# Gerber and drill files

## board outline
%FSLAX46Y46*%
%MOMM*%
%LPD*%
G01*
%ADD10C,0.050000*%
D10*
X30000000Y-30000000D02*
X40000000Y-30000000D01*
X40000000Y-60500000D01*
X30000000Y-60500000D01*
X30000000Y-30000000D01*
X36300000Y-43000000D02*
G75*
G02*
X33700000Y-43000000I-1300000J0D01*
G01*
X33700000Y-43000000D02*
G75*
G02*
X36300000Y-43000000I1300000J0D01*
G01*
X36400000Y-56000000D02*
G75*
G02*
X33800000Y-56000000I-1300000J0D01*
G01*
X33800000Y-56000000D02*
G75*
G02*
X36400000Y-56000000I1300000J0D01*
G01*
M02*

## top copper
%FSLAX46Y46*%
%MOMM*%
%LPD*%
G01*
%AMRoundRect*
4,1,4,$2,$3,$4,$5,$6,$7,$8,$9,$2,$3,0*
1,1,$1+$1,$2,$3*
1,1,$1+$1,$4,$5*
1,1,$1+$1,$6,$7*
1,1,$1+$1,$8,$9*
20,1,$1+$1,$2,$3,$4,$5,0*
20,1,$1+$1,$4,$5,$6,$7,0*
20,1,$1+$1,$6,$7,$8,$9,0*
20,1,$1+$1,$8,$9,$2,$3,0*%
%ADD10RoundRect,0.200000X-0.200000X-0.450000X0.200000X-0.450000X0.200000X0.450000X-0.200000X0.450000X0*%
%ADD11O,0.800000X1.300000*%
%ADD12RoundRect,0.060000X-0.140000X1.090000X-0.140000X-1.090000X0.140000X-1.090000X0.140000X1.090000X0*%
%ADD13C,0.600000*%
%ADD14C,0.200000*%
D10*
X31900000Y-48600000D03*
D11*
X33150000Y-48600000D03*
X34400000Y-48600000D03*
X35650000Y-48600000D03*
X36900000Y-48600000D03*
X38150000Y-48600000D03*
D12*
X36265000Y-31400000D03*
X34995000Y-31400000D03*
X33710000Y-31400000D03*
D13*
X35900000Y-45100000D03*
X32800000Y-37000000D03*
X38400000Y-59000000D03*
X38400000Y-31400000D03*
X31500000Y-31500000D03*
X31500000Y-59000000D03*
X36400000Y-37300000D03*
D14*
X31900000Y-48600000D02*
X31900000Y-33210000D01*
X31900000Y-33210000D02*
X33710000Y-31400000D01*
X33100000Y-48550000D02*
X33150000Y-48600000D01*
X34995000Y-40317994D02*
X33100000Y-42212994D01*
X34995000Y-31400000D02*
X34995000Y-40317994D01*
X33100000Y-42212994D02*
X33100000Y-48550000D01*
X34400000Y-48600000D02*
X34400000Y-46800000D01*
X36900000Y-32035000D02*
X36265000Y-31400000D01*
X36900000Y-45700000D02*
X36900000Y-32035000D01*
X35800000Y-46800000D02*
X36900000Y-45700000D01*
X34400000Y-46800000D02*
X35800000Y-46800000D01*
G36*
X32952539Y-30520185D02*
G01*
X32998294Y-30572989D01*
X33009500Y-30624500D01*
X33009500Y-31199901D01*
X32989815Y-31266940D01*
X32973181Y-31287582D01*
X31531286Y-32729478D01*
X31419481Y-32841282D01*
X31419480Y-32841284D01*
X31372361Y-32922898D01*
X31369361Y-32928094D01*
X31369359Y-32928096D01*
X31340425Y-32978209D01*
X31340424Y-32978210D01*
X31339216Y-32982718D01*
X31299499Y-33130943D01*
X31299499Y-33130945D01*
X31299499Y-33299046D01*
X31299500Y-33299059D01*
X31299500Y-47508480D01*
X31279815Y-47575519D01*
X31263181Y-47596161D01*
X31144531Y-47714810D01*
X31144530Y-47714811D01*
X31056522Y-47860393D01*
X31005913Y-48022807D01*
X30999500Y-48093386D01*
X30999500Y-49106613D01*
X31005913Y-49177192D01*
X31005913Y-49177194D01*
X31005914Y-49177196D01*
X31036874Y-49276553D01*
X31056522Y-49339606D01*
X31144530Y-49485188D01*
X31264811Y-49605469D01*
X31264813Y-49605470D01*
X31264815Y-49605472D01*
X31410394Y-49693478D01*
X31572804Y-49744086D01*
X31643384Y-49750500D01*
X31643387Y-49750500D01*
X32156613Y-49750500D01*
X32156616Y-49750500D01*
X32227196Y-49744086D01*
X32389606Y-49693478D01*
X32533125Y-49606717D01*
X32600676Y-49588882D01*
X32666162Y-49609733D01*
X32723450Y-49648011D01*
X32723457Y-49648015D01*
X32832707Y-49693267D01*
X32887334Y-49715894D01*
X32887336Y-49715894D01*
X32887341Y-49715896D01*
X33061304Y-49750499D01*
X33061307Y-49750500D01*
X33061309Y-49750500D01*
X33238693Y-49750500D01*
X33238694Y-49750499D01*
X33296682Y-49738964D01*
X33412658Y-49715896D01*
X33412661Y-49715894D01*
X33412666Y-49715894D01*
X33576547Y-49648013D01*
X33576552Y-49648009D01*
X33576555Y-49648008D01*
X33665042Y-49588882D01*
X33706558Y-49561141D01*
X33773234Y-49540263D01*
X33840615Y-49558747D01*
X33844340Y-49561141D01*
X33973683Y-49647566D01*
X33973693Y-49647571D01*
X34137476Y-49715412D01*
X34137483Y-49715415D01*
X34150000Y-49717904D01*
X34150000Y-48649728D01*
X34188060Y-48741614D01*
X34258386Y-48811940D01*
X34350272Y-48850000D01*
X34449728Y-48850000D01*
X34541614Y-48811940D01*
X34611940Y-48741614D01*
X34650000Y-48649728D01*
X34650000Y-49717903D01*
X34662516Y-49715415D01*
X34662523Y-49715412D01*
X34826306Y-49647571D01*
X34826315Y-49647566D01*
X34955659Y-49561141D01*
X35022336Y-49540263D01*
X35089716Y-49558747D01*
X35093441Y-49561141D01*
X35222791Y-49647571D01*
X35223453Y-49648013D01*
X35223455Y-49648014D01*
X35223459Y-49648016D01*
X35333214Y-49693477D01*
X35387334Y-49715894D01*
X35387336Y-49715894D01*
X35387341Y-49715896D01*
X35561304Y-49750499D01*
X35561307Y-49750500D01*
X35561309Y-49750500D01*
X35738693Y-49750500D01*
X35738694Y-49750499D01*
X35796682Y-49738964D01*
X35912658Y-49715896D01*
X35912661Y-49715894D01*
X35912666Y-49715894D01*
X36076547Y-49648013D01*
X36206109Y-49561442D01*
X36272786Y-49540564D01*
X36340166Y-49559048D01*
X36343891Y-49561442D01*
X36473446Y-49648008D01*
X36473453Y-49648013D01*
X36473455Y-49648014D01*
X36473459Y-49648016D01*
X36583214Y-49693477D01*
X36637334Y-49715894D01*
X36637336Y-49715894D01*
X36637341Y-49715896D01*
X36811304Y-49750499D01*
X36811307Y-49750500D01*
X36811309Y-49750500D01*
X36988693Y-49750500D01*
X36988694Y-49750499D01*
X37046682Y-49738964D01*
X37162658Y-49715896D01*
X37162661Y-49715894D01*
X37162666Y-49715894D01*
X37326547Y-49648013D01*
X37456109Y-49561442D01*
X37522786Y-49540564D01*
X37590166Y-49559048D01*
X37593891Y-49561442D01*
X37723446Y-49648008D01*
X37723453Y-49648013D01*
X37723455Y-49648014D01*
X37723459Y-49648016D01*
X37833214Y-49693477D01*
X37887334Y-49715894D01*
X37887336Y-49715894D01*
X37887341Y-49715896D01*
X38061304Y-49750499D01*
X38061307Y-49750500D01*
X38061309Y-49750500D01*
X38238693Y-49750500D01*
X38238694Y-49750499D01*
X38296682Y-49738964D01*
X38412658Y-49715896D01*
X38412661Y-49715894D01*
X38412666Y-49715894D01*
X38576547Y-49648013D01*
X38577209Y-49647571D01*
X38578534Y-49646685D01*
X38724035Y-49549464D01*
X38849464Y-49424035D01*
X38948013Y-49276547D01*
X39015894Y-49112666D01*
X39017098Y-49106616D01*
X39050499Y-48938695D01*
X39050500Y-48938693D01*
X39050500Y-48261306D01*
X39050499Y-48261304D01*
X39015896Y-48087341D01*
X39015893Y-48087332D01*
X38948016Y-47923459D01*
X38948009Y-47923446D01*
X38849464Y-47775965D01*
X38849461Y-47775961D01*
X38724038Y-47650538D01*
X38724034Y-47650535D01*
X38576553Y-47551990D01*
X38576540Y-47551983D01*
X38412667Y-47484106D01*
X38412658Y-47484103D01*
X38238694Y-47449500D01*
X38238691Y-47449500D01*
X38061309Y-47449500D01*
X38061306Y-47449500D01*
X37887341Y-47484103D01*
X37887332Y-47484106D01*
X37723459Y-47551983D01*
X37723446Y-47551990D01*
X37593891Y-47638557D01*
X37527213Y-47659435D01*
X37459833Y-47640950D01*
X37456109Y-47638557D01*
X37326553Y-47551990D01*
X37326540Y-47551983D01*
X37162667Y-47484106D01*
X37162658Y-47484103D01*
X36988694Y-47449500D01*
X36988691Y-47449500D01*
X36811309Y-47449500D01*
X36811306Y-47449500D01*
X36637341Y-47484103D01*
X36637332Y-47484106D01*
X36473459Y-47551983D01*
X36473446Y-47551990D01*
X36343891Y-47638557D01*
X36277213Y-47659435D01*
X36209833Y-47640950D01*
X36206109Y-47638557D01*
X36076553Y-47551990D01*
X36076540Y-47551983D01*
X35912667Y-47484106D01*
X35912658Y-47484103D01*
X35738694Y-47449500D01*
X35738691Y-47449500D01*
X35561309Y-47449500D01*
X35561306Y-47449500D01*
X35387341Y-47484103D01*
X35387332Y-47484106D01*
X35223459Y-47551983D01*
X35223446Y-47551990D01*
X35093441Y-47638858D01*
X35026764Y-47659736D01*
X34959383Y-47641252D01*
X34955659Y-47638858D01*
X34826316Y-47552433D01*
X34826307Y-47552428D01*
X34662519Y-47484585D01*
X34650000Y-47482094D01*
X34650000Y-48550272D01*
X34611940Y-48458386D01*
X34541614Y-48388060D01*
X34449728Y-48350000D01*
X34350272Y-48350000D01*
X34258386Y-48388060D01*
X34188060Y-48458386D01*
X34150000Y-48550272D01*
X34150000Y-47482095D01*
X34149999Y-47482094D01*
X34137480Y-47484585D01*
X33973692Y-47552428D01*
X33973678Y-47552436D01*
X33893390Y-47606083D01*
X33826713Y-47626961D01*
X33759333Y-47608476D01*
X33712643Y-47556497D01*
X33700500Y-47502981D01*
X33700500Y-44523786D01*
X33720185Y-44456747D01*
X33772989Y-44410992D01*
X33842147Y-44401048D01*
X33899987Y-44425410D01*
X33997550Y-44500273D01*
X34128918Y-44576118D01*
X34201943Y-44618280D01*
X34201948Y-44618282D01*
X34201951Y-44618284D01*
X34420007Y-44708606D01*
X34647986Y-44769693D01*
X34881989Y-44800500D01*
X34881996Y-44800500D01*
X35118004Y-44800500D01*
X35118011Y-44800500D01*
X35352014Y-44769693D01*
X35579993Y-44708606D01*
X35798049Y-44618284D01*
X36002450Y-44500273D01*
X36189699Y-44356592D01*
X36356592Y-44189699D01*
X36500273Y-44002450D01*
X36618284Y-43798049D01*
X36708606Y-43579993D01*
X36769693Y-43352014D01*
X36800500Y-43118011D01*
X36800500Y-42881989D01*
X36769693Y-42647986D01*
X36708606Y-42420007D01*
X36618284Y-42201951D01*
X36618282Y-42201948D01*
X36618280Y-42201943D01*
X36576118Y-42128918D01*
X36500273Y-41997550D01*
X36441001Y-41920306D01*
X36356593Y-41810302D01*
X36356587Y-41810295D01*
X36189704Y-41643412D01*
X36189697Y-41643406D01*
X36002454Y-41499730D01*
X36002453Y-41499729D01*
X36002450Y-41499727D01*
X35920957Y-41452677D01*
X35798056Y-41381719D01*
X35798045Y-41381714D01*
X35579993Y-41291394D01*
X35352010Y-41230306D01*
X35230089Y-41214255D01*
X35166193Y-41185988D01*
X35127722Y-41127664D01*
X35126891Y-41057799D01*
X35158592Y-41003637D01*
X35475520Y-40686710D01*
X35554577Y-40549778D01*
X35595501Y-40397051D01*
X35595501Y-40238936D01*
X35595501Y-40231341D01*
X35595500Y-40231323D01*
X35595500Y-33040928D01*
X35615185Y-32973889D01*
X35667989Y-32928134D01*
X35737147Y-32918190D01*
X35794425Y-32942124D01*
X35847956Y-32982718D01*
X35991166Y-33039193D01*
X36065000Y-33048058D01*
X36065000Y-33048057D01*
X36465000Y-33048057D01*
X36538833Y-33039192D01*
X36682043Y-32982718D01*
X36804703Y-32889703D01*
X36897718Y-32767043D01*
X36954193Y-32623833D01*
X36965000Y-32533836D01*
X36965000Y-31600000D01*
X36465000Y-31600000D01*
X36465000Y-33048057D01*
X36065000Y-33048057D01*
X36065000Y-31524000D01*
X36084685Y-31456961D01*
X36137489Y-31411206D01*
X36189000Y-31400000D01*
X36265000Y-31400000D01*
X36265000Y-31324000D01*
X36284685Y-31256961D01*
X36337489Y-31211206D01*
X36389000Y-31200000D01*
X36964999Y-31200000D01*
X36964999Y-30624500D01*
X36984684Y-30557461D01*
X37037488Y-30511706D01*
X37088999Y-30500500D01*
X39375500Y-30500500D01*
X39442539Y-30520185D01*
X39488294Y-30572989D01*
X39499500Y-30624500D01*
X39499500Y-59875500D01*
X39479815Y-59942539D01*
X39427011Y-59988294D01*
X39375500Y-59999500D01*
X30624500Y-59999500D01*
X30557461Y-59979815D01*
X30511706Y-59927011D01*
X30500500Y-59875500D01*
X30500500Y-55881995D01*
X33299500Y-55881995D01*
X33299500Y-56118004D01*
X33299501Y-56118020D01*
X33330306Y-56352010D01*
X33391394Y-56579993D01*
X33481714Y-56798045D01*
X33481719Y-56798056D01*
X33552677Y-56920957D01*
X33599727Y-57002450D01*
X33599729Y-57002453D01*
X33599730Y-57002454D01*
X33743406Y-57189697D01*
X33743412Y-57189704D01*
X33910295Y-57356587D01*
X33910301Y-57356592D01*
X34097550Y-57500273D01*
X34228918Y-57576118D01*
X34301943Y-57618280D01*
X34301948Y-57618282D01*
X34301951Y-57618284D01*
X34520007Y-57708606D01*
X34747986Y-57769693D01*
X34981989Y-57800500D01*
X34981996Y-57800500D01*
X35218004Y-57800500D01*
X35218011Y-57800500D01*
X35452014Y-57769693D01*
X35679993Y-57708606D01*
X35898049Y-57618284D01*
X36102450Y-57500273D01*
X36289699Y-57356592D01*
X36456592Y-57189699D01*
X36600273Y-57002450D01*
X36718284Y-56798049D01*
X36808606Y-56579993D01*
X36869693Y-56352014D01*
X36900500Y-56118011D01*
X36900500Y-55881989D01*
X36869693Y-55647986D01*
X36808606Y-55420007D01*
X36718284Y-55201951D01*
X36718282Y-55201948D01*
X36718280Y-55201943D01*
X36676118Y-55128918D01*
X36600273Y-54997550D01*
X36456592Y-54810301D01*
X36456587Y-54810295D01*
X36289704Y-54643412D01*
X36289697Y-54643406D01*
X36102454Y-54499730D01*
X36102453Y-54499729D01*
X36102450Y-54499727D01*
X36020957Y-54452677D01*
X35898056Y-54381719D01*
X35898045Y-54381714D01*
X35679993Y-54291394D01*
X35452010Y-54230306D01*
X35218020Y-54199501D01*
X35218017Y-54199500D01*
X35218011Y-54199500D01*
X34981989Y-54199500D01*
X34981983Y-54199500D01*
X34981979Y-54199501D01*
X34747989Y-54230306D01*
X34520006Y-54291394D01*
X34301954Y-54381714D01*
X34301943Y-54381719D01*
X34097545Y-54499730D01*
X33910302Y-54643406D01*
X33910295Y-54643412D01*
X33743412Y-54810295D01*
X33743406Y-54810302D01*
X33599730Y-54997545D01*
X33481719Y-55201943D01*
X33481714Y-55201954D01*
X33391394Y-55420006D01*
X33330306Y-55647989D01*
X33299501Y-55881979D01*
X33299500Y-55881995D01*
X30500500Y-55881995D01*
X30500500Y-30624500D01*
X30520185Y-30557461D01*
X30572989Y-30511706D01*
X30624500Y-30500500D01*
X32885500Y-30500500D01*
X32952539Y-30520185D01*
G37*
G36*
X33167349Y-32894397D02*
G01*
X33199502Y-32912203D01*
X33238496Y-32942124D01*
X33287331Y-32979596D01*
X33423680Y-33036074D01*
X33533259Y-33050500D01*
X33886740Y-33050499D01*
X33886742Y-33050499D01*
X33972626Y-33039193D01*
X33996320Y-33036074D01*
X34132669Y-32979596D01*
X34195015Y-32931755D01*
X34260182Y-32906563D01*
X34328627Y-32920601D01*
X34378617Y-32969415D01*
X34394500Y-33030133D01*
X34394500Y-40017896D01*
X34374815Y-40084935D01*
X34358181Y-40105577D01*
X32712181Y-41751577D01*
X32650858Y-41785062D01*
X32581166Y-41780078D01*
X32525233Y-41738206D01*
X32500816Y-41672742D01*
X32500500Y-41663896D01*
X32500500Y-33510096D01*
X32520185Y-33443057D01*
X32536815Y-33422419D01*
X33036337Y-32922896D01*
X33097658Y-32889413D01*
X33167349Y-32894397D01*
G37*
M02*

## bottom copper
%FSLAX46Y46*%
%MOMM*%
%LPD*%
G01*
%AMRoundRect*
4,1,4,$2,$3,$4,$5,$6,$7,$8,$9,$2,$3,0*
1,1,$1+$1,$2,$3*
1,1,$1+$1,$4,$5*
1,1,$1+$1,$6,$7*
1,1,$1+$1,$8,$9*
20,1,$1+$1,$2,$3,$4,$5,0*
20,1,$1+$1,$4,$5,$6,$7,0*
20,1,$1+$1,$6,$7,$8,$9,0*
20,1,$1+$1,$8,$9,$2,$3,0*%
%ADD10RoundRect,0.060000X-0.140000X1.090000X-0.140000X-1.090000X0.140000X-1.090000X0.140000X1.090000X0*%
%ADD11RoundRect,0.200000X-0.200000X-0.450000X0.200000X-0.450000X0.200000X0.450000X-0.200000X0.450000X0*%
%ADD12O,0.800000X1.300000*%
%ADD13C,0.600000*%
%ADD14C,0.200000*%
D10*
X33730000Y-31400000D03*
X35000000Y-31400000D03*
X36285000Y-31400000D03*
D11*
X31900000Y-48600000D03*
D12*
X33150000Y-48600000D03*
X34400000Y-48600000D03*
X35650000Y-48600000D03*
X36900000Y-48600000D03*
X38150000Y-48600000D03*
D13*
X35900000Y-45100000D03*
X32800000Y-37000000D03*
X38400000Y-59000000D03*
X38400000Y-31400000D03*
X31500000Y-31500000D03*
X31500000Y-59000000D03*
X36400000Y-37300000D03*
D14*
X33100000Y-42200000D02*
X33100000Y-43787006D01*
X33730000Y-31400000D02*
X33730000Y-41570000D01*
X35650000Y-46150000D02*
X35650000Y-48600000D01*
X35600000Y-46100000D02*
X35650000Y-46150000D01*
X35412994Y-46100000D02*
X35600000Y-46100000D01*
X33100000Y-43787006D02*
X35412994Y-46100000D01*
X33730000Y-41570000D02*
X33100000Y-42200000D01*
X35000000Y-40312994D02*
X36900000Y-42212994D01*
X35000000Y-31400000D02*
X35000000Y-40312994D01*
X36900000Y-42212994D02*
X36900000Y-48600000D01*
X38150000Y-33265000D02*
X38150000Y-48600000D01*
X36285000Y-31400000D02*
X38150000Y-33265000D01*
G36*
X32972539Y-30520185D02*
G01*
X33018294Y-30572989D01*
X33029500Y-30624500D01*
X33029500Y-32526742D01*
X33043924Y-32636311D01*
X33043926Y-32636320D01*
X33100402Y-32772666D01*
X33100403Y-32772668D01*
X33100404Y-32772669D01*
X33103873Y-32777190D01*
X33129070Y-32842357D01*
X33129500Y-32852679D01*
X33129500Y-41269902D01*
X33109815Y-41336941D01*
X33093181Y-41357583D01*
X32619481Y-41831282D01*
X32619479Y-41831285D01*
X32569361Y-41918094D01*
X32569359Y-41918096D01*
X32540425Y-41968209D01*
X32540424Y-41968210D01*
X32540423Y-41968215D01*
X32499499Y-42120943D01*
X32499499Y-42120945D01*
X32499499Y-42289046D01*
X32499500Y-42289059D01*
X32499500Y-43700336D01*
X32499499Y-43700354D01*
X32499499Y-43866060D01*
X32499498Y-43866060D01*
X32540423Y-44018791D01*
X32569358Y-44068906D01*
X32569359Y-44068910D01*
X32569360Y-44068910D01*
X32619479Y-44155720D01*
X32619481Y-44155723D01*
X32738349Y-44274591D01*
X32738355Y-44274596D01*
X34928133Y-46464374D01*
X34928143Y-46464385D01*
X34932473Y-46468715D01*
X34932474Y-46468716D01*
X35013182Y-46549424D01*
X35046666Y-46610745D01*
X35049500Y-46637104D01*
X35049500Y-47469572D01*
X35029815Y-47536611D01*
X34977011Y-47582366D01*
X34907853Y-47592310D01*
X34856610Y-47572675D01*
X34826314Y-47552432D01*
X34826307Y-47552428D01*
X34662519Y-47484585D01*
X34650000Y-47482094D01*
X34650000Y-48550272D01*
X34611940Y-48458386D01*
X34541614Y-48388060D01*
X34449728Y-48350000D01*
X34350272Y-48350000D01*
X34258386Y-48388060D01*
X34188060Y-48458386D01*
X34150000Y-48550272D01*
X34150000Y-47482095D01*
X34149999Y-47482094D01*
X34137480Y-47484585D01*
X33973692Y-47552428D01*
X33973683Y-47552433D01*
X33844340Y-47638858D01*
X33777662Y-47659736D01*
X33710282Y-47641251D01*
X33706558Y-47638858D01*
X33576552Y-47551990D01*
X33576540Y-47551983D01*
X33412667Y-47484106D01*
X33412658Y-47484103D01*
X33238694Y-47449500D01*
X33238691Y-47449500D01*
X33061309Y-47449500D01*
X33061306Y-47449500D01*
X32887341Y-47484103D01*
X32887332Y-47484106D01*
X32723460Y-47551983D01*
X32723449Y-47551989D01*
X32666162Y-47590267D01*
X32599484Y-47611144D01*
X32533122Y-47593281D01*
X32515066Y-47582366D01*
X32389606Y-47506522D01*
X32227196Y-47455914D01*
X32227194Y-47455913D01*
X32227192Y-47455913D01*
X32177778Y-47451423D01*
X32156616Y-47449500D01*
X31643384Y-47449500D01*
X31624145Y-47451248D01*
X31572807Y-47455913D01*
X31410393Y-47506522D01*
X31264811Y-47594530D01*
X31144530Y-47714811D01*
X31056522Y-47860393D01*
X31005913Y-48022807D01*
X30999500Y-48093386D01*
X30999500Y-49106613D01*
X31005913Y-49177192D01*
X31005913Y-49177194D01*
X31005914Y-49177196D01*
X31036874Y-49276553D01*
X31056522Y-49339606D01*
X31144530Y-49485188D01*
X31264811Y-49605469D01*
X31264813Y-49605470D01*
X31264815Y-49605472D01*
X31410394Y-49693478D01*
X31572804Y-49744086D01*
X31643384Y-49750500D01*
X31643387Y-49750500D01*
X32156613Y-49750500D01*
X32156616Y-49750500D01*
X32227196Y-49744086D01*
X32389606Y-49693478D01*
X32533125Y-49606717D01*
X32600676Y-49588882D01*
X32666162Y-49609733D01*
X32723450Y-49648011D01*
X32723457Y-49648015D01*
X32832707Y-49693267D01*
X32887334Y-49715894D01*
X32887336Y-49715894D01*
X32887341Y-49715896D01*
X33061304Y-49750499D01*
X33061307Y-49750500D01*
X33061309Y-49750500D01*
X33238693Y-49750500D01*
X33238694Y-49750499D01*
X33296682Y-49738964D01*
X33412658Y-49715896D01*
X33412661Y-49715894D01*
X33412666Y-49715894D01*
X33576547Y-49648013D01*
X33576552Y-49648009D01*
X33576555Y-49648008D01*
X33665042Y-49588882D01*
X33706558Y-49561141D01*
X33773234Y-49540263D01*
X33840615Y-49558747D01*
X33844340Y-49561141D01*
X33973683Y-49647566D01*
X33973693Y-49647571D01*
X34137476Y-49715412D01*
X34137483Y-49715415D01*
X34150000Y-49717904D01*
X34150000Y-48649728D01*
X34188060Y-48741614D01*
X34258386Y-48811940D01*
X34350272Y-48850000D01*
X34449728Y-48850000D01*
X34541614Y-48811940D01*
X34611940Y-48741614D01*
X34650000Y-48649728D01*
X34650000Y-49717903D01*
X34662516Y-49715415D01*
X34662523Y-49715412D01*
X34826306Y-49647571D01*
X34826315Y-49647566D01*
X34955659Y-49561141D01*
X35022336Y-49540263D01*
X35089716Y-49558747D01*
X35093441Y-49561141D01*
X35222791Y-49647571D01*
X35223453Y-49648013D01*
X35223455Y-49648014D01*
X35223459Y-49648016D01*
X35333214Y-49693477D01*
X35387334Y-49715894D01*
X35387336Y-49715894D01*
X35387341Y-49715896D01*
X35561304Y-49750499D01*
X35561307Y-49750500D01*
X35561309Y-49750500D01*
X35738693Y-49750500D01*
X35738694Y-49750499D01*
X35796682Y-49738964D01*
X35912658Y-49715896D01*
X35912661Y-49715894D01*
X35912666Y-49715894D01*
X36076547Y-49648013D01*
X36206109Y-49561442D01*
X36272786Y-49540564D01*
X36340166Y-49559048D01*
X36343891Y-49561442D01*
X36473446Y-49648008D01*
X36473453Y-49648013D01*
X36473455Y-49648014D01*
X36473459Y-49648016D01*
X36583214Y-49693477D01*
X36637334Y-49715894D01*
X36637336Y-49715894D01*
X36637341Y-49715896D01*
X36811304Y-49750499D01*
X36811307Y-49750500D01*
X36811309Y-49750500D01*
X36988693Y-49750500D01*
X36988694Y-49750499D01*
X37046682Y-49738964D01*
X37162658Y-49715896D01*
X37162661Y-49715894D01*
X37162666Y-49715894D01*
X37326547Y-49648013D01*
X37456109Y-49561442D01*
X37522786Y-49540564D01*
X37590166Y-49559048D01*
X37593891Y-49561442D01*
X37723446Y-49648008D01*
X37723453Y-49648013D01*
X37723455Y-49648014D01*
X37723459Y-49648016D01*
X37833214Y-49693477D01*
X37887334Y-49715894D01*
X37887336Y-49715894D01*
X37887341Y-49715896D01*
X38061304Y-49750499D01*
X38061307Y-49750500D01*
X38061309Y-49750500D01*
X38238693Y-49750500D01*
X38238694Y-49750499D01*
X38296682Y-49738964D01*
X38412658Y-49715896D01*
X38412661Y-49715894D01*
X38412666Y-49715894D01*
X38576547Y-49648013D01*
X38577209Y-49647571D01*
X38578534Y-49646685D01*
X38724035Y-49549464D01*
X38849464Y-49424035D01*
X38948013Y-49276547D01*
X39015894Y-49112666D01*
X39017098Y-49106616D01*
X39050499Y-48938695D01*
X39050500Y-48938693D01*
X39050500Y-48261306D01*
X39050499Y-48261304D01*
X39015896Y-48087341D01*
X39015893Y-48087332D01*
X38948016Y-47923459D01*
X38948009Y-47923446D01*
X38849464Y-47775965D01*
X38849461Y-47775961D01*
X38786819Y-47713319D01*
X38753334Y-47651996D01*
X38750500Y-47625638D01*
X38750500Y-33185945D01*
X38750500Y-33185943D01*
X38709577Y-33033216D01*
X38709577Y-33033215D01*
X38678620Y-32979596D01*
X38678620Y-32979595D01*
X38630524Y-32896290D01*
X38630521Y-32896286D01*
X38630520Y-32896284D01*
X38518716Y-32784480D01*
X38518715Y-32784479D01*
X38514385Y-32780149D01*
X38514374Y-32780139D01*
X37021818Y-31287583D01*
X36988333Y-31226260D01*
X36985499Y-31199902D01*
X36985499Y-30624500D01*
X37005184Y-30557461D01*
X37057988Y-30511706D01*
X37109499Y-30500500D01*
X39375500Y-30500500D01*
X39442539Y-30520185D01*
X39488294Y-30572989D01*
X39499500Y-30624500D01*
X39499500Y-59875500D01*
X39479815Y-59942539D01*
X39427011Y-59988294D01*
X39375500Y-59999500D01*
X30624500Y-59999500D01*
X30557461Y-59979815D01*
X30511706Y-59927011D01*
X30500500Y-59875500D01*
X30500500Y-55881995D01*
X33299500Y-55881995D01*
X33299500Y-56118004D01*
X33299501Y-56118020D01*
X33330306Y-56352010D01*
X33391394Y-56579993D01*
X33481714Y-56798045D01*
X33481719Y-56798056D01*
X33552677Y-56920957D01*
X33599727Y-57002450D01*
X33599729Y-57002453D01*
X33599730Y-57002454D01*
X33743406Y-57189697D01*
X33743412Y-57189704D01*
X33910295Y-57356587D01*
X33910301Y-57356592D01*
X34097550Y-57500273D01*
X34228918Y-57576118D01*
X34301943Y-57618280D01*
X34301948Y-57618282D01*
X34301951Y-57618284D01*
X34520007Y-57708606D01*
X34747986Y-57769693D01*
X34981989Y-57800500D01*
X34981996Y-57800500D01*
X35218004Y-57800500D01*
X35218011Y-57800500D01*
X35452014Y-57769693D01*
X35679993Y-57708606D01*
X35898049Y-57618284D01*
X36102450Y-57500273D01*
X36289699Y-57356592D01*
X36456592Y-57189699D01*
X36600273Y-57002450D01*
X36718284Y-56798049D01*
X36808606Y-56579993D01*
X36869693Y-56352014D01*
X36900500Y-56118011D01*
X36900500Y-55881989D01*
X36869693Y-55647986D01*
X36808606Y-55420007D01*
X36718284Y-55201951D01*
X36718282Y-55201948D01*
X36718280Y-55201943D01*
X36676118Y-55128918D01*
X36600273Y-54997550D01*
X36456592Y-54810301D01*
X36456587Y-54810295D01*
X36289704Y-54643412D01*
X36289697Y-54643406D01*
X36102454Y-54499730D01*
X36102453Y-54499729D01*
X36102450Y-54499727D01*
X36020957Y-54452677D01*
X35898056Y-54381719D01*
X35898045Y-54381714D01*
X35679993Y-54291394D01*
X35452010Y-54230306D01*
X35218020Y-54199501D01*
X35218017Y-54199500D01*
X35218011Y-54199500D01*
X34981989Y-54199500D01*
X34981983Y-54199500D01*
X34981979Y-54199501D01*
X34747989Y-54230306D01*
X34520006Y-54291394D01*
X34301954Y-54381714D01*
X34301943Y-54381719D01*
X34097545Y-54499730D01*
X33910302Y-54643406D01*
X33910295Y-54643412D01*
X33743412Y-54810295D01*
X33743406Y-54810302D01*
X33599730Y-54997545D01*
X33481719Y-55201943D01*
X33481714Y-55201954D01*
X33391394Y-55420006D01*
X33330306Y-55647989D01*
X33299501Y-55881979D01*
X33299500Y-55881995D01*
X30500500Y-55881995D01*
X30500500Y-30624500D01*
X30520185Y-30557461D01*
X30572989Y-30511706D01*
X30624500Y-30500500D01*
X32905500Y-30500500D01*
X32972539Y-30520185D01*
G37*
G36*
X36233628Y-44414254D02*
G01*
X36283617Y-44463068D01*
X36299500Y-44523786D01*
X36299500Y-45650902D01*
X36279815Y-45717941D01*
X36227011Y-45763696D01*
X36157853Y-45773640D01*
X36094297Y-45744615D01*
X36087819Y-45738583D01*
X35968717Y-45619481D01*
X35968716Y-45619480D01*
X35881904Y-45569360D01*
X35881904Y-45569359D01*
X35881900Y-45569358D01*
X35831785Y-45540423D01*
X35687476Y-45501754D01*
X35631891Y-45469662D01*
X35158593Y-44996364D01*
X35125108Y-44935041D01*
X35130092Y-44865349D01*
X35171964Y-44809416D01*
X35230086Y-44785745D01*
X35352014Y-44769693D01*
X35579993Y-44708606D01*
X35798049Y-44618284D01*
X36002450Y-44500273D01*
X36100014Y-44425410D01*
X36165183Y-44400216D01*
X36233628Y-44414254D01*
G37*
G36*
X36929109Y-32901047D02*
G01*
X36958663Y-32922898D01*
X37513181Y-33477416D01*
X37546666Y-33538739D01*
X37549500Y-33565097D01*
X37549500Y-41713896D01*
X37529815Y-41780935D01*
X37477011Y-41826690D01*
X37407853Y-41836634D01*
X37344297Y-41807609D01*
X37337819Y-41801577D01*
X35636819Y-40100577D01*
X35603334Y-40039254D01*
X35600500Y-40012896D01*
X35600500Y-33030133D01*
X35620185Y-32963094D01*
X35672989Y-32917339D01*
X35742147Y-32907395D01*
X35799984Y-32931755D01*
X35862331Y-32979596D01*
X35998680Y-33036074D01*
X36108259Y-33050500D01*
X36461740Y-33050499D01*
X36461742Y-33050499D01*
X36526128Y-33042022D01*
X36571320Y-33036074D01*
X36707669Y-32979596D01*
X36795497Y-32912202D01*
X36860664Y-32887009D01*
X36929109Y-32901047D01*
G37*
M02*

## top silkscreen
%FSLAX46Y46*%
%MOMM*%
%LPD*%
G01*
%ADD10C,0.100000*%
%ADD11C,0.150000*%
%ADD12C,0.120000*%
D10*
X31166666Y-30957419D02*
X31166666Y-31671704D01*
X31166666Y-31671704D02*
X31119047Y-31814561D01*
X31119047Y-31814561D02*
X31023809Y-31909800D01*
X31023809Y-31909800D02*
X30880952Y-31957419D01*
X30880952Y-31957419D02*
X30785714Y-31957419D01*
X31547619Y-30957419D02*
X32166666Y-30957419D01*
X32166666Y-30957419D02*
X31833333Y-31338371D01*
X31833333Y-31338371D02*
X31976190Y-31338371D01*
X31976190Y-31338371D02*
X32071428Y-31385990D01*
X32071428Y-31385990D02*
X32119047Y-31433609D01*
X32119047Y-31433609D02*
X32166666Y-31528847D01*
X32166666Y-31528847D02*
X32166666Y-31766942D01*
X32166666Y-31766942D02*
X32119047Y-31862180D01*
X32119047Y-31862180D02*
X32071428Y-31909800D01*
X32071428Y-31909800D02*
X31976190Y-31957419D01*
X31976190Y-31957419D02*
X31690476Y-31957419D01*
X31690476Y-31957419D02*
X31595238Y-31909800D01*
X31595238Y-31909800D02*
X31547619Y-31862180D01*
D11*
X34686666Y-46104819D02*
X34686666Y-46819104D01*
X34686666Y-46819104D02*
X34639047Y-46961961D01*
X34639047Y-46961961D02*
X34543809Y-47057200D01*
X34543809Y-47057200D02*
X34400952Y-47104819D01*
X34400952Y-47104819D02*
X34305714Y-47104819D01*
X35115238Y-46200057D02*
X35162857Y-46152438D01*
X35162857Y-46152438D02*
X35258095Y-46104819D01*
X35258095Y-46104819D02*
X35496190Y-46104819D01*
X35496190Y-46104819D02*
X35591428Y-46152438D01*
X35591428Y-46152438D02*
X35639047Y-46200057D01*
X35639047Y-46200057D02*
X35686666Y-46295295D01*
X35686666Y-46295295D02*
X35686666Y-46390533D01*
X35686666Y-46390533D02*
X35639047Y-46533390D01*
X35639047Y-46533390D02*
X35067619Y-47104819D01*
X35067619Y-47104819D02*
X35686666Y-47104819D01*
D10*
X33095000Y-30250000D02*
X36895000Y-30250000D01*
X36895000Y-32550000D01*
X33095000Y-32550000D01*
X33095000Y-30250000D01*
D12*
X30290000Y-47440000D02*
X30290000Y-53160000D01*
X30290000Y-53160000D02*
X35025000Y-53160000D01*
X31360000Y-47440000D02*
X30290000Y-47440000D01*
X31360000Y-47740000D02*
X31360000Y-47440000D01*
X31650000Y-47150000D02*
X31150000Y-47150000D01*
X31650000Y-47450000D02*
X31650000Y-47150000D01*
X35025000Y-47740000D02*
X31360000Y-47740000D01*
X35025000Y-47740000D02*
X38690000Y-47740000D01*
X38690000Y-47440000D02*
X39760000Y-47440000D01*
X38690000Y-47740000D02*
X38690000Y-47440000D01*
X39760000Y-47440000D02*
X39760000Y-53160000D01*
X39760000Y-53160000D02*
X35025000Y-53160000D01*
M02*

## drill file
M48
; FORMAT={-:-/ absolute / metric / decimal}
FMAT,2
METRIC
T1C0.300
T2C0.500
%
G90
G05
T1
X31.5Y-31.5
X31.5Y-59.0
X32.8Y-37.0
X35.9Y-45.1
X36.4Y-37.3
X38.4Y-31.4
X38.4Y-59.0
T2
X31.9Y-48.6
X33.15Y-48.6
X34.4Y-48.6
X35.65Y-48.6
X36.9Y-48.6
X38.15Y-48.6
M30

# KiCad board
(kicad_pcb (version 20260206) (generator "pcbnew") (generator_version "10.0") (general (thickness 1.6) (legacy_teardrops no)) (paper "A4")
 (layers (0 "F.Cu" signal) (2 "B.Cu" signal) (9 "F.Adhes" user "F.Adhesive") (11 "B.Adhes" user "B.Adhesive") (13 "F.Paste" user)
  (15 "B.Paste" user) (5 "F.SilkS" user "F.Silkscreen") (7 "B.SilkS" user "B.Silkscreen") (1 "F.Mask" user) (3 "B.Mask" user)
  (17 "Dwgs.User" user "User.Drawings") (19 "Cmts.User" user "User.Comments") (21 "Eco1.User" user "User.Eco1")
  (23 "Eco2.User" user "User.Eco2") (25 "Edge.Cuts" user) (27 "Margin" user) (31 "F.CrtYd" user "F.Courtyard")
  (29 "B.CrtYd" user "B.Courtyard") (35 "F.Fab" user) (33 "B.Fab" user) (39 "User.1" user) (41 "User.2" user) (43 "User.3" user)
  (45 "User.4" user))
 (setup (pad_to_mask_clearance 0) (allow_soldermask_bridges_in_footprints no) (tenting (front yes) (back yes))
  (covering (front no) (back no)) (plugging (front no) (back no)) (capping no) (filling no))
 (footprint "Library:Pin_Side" (layer "F.Cu") (at 33.095 30.25 -90)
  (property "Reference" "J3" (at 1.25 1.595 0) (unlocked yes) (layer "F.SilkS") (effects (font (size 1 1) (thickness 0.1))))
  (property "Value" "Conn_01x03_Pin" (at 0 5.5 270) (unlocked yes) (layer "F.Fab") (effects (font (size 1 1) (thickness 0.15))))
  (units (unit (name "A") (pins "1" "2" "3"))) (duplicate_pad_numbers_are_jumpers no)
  (fp_rect (start 0 -3.8) (end 2.3 0) (stroke (width 0.1) (type default)) (fill no) (layer "F.SilkS"))
  (pad "1" smd roundrect (at 1.15 -0.635 270) (size 2.3 0.4) (layers "*.Mask" "B.Cu") (roundrect_rratio 0.15) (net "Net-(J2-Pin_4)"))
  (pad "2" smd roundrect (at 1.15 -1.905 270) (size 2.3 0.4) (layers "*.Mask" "B.Cu") (roundrect_rratio 0.15) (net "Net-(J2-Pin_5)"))
  (pad "3" smd roundrect (at 1.15 -3.19 270) (size 2.3 0.4) (layers "*.Mask" "B.Cu") (roundrect_rratio 0.15) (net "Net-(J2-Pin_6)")))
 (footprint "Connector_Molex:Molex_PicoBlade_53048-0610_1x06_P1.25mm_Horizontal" (layer "F.Cu") (at 31.9 48.6)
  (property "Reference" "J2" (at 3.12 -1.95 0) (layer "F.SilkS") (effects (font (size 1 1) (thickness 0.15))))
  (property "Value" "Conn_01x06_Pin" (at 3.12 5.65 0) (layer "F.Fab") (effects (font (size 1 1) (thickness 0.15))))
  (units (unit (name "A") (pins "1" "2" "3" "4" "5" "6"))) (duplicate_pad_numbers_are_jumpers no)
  (fp_line (start -1.61 -1.16) (end -1.61 4.56) (stroke (width 0.12) (type solid)) (layer "F.SilkS"))
  (fp_line (start -1.61 4.56) (end 3.125 4.56) (stroke (width 0.12) (type solid)) (layer "F.SilkS"))
  (fp_line (start -0.54 -1.16) (end -1.61 -1.16) (stroke (width 0.12) (type solid)) (layer "F.SilkS"))
  (fp_line (start -0.54 -0.86) (end -0.54 -1.16) (stroke (width 0.12) (type solid)) (layer "F.SilkS"))
  (fp_line (start -0.25 -1.45) (end -0.75 -1.45) (stroke (width 0.12) (type solid)) (layer "F.SilkS"))
  (fp_line (start -0.25 -1.15) (end -0.25 -1.45) (stroke (width 0.12) (type solid)) (layer "F.SilkS"))
  (fp_line (start 3.125 -0.86) (end -0.54 -0.86) (stroke (width 0.12) (type solid)) (layer "F.SilkS"))
  (fp_line (start 3.125 -0.86) (end 6.79 -0.86) (stroke (width 0.12) (type solid)) (layer "F.SilkS"))
  (fp_line (start 6.79 -1.16) (end 7.86 -1.16) (stroke (width 0.12) (type solid)) (layer "F.SilkS"))
  (fp_line (start 6.79 -0.86) (end 6.79 -1.16) (stroke (width 0.12) (type solid)) (layer "F.SilkS"))
  (fp_line (start 7.86 -1.16) (end 7.86 4.56) (stroke (width 0.12) (type solid)) (layer "F.SilkS"))
  (fp_line (start 7.86 4.56) (end 3.125 4.56) (stroke (width 0.12) (type solid)) (layer "F.SilkS"))
  (pad "1" thru_hole roundrect (at 0 0) (size 0.8 1.3) (drill 0.5) (layers "*.Cu" "*.Mask") (remove_unused_layers no)
   (roundrect_rratio 0.25) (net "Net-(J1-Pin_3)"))
  (pad "2" thru_hole oval (at 1.25 0) (size 0.8 1.3) (drill 0.5) (layers "*.Cu" "*.Mask") (remove_unused_layers no) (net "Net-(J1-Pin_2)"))
  (pad "3" thru_hole oval (at 2.5 0) (size 0.8 1.3) (drill 0.5) (layers "*.Cu" "*.Mask") (remove_unused_layers no) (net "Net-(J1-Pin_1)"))
  (pad "4" thru_hole oval (at 3.75 0) (size 0.8 1.3) (drill 0.5) (layers "*.Cu" "*.Mask") (remove_unused_layers no) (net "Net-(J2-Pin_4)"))
  (pad "5" thru_hole oval (at 5 0) (size 0.8 1.3) (drill 0.5) (layers "*.Cu" "*.Mask") (remove_unused_layers no) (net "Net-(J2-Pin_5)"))
  (pad "6" thru_hole oval (at 6.25 0) (size 0.8 1.3) (drill 0.5) (layers "*.Cu" "*.Mask") (remove_unused_layers no) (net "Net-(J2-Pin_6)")))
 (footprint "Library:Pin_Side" (layer "B.Cu") (at 36.9 30.25 -90)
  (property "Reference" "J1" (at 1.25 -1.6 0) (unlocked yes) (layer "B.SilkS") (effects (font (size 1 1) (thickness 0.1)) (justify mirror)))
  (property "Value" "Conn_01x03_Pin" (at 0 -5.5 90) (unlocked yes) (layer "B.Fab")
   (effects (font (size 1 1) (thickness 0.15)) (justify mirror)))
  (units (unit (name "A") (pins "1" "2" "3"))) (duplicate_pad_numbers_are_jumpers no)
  (pad "1" smd roundrect (at 1.15 0.635 270) (size 2.3 0.4) (layers "*.Mask" "F.Cu") (roundrect_rratio 0.15) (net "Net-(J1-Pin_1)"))
  (pad "2" smd roundrect (at 1.15 1.905 270) (size 2.3 0.4) (layers "*.Mask" "F.Cu") (roundrect_rratio 0.15) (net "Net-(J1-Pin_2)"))
  (pad "3" smd roundrect (at 1.15 3.19 270) (size 2.3 0.4) (layers "*.Mask" "F.Cu") (roundrect_rratio 0.15) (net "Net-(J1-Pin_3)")))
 (gr_rect (start 30 30) (end 40 60.5) (stroke (width 0.05) (type default)) (fill no) (layer "Edge.Cuts"))
 (gr_circle (center 35 43) (end 36.3 43) (stroke (width 0.05) (type default)) (fill no) (layer "Edge.Cuts"))
 (gr_circle (center 35.1 56) (end 36.4 56) (stroke (width 0.05) (type default)) (fill no) (layer "Edge.Cuts"))
 (segment (start 33.1 42.2) (end 33.1 43.787006) (width 0.2) (layer "B.Cu") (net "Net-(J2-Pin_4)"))
 (segment (start 33.73 31.4) (end 33.73 41.57) (width 0.2) (layer "B.Cu") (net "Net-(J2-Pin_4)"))
 (segment (start 35.65 46.15) (end 35.65 48.6) (width 0.2) (layer "B.Cu") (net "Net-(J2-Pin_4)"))
 (segment (start 35.6 46.1) (end 35.65 46.15) (width 0.2) (layer "B.Cu") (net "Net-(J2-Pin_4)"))
 (segment (start 35.412994 46.1) (end 35.6 46.1) (width 0.2) (layer "B.Cu") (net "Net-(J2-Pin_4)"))
 (segment (start 33.1 43.787006) (end 35.412994 46.1) (width 0.2) (layer "B.Cu") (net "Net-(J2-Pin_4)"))
 (segment (start 33.73 41.57) (end 33.1 42.2) (width 0.2) (layer "B.Cu") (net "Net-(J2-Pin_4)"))
 (segment (start 35 40.312994) (end 36.9 42.212994) (width 0.2) (layer "B.Cu") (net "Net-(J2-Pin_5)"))
 (segment (start 35 31.4) (end 35 40.312994) (width 0.2) (layer "B.Cu") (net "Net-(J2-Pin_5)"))
 (segment (start 36.9 42.212994) (end 36.9 48.6) (width 0.2) (layer "B.Cu") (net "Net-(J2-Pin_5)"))
 (segment (start 38.15 33.265) (end 38.15 48.6) (width 0.2) (layer "B.Cu") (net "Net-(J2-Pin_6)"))
 (segment (start 36.285 31.4) (end 38.15 33.265) (width 0.2) (layer "B.Cu") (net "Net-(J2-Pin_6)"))
 (segment (start 31.9 48.6) (end 31.9 33.21) (width 0.2) (layer "F.Cu") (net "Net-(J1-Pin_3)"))
 (segment (start 31.9 33.21) (end 33.71 31.4) (width 0.2) (layer "F.Cu") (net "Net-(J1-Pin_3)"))
 (segment (start 33.1 48.55) (end 33.15 48.6) (width 0.2) (layer "F.Cu") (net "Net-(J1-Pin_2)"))
 (segment (start 34.995 40.317994) (end 33.1 42.212994) (width 0.2) (layer "F.Cu") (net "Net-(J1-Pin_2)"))
 (segment (start 34.995 31.4) (end 34.995 40.317994) (width 0.2) (layer "F.Cu") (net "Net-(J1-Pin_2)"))
 (segment (start 33.1 42.212994) (end 33.1 48.55) (width 0.2) (layer "F.Cu") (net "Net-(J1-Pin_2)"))
 (segment (start 34.4 48.6) (end 34.4 46.8) (width 0.2) (layer "F.Cu") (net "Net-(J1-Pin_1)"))
 (segment (start 36.9 32.035) (end 36.265 31.4) (width 0.2) (layer "F.Cu") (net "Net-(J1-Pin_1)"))
 (segment (start 36.9 45.7) (end 36.9 32.035) (width 0.2) (layer "F.Cu") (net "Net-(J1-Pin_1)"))
 (segment (start 35.8 46.8) (end 36.9 45.7) (width 0.2) (layer "F.Cu") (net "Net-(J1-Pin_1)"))
 (segment (start 34.4 46.8) (end 35.8 46.8) (width 0.2) (layer "F.Cu") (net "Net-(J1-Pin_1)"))
 (via (at 35.9 45.1) (size 0.6) (drill 0.3) (layers "F.Cu" "B.Cu") (free yes) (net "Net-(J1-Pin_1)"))
 (via (at 32.8 37) (size 0.6) (drill 0.3) (layers "F.Cu" "B.Cu") (free yes) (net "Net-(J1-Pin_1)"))
 (via (at 38.4 59) (size 0.6) (drill 0.3) (layers "F.Cu" "B.Cu") (free yes) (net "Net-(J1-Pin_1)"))
 (via (at 38.4 31.4) (size 0.6) (drill 0.3) (layers "F.Cu" "B.Cu") (free yes) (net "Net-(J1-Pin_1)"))
 (via (at 31.5 31.5) (size 0.6) (drill 0.3) (layers "F.Cu" "B.Cu") (free yes) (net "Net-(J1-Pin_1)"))
 (via (at 31.5 59) (size 0.6) (drill 0.3) (layers "F.Cu" "B.Cu") (free yes) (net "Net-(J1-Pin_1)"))
 (via (at 36.4 37.3) (size 0.6) (drill 0.3) (layers "F.Cu" "B.Cu") (free yes) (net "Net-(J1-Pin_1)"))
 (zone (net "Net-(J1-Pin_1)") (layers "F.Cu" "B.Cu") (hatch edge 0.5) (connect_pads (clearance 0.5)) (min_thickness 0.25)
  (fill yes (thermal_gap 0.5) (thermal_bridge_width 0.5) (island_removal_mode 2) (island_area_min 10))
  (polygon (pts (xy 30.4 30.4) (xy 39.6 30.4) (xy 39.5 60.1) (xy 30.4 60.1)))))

